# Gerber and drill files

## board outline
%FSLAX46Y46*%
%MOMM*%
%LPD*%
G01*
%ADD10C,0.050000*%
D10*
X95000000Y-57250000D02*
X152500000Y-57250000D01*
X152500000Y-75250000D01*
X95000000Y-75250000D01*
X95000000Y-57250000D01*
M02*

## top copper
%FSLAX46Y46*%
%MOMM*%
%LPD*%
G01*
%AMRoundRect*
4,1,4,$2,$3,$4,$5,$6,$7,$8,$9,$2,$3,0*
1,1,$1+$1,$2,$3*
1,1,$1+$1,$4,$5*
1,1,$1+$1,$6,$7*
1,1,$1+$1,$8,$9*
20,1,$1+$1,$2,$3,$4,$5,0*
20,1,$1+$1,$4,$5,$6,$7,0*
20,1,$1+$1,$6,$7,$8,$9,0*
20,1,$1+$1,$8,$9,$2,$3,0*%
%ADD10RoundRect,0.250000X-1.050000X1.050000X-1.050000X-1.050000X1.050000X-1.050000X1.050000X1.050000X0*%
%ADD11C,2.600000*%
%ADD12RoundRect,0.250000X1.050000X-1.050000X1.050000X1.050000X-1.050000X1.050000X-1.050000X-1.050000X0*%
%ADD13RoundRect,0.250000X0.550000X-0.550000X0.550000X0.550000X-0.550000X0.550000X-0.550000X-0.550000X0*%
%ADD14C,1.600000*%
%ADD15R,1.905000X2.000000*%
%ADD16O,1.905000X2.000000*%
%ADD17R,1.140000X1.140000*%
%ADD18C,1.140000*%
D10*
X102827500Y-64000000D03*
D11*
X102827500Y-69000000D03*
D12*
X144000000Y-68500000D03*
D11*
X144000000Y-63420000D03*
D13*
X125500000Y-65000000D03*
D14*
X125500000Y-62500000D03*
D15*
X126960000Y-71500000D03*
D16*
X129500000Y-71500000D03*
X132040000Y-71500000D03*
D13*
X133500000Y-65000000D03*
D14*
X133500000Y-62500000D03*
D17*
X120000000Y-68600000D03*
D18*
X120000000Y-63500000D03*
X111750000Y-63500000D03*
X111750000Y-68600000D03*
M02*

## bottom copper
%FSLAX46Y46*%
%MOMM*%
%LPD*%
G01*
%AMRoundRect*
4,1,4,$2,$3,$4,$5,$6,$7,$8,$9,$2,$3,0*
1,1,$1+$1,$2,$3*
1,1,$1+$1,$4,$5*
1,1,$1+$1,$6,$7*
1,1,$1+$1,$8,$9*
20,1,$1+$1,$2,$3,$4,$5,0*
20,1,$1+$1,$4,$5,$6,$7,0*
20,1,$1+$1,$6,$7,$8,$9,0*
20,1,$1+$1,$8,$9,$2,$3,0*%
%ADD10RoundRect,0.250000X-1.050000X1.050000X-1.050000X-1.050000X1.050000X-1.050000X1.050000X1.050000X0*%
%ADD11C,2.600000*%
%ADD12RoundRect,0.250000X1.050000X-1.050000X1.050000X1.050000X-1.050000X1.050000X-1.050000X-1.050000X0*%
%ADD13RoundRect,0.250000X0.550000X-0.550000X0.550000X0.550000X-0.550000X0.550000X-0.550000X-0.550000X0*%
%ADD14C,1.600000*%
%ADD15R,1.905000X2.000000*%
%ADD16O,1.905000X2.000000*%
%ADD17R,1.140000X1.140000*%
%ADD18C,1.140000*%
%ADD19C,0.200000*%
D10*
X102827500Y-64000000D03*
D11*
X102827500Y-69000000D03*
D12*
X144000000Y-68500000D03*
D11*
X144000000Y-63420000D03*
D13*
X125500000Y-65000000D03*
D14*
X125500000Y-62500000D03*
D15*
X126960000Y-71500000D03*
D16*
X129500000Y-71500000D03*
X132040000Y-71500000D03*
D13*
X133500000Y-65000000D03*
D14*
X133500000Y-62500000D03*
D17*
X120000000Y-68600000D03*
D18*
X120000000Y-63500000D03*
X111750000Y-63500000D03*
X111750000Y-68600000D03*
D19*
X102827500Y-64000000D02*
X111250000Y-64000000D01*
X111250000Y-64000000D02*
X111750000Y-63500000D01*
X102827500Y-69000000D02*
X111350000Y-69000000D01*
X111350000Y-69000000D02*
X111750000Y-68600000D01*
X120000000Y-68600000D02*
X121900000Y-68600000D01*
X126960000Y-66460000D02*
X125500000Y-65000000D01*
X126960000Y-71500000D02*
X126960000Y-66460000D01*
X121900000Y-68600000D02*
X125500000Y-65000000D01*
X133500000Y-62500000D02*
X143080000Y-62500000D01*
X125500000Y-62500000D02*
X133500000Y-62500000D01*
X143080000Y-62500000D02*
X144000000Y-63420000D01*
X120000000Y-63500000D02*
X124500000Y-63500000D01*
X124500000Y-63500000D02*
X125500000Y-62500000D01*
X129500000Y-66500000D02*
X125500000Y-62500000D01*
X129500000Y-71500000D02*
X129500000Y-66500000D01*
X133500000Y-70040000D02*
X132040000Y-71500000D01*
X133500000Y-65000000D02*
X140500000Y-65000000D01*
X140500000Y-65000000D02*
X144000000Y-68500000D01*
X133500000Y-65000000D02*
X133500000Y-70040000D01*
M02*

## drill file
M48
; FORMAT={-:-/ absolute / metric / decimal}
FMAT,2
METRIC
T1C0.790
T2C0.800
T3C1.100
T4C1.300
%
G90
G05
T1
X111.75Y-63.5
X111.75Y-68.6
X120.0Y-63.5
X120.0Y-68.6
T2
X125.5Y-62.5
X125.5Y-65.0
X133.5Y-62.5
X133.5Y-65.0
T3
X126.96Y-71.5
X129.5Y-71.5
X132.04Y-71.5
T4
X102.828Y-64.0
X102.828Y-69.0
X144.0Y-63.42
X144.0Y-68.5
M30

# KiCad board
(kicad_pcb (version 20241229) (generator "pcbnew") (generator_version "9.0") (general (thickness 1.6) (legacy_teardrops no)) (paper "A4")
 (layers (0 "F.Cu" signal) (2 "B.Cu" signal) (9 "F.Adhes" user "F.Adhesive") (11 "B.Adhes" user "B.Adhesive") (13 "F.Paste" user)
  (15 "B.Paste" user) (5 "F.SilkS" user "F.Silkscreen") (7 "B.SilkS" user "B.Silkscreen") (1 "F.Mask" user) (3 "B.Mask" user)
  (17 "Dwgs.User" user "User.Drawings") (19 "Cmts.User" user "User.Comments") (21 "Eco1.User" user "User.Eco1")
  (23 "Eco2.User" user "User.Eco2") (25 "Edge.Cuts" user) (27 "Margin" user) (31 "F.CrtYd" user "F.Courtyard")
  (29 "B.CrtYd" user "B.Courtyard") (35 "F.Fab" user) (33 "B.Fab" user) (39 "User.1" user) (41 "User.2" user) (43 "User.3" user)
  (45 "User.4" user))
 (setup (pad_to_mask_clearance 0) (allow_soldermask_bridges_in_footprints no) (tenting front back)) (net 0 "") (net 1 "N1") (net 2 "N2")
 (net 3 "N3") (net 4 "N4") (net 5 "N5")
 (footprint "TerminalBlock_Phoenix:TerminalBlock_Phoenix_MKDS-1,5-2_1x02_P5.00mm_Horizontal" (layer "F.Cu") (at 102.8275 64 -90)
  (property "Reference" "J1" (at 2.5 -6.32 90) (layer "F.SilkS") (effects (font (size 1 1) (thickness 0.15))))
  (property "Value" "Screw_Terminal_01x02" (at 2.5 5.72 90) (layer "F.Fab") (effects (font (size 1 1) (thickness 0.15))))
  (pad "1" thru_hole roundrect (at 0 0 270) (size 2.6 2.6) (drill 1.3) (layers "*.Cu" "*.Mask") (remove_unused_layers no)
   (roundrect_rratio 0.096154) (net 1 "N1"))
  (pad "2" thru_hole circle (at 5 0 270) (size 2.6 2.6) (drill 1.3) (layers "*.Cu" "*.Mask") (remove_unused_layers no) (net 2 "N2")))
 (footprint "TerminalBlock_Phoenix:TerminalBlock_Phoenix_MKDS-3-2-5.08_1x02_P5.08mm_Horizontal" (layer "F.Cu") (at 144 68.5 90)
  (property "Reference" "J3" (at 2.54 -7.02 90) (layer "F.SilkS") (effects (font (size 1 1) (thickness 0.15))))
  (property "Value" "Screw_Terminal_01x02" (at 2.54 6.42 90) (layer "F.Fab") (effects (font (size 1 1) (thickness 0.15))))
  (pad "1" thru_hole roundrect (at 0 0 90) (size 2.6 2.6) (drill 1.3) (layers "*.Cu" "*.Mask") (remove_unused_layers no)
   (roundrect_rratio 0.096154) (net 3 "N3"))
  (pad "2" thru_hole circle (at 5.08 0 90) (size 2.6 2.6) (drill 1.3) (layers "*.Cu" "*.Mask") (remove_unused_layers no) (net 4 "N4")))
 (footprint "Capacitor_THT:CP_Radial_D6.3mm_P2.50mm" (layer "F.Cu") (at 125.5 65 90)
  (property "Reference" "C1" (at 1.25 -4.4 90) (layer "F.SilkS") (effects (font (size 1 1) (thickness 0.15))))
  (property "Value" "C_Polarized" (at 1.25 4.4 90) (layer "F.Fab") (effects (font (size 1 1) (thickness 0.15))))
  (pad "1" thru_hole roundrect (at 0 0 90) (size 1.6 1.6) (drill 0.8) (layers "*.Cu" "*.Mask") (remove_unused_layers no)
   (roundrect_rratio 0.15625) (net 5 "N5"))
  (pad "2" thru_hole circle (at 2.5 0 90) (size 1.6 1.6) (drill 0.8) (layers "*.Cu" "*.Mask") (remove_unused_layers no) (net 4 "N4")))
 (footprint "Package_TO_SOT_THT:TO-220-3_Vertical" (layer "F.Cu") (at 126.96 71.5)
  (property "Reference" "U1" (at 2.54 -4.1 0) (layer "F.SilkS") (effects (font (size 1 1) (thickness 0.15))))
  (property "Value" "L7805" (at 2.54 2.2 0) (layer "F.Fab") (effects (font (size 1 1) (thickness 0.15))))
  (pad "1" thru_hole rect (at 0 0) (size 1.905 2) (drill 1.1) (layers "*.Cu" "*.Mask") (remove_unused_layers no) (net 5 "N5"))
  (pad "2" thru_hole oval (at 2.54 0) (size 1.905 2) (drill 1.1) (layers "*.Cu" "*.Mask") (remove_unused_layers no) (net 4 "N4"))
  (pad "3" thru_hole oval (at 5.08 0) (size 1.905 2) (drill 1.1) (layers "*.Cu" "*.Mask") (remove_unused_layers no) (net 3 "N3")))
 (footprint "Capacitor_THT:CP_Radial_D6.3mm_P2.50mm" (layer "F.Cu") (at 133.5 65 90)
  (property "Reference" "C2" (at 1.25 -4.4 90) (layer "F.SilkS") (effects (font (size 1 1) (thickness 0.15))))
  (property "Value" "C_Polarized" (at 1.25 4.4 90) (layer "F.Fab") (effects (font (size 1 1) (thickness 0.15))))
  (pad "1" thru_hole roundrect (at 0 0 90) (size 1.6 1.6) (drill 0.8) (layers "*.Cu" "*.Mask") (remove_unused_layers no)
   (roundrect_rratio 0.15625) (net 3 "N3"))
  (pad "2" thru_hole circle (at 2.5 0 90) (size 1.6 1.6) (drill 0.8) (layers "*.Cu" "*.Mask") (remove_unused_layers no) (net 4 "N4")))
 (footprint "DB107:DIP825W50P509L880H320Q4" (layer "F.Cu") (at 115.875 66.05 180)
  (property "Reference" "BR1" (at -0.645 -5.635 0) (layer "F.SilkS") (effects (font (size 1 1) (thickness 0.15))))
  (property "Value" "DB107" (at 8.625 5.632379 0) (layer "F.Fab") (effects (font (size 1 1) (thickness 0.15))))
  (pad "1" thru_hole rect (at -4.125 -2.55 180) (size 1.14 1.14) (drill 0.79) (layers "*.Cu" "*.Mask") (remove_unused_layers no)
   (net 5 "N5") (solder_mask_margin 0.102))
  (pad "2" thru_hole circle (at -4.125 2.55 180) (size 1.14 1.14) (drill 0.79) (layers "*.Cu" "*.Mask") (remove_unused_layers no)
   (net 4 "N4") (solder_mask_margin 0.102))
  (pad "3" thru_hole circle (at 4.125 2.55 180) (size 1.14 1.14) (drill 0.79) (layers "*.Cu" "*.Mask") (remove_unused_layers no)
   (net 1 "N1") (solder_mask_margin 0.102))
  (pad "4" thru_hole circle (at 4.125 -2.55 180) (size 1.14 1.14) (drill 0.79) (layers "*.Cu" "*.Mask") (remove_unused_layers no)
   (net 2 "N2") (solder_mask_margin 0.102)))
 (gr_rect (start 95 57.25) (end 152.5 75.25) (stroke (width 0.05) (type default)) (fill no) (layer "Edge.Cuts"))
 (segment (start 102.8275 64) (end 111.25 64) (width 0.2) (layer "B.Cu") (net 1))
 (segment (start 111.25 64) (end 111.75 63.5) (width 0.2) (layer "B.Cu") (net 1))
 (segment (start 102.8275 69) (end 111.35 69) (width 0.2) (layer "B.Cu") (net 2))
 (segment (start 111.35 69) (end 111.75 68.6) (width 0.2) (layer "B.Cu") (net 2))
 (segment (start 120 68.6) (end 121.9 68.6) (width 0.2) (layer "B.Cu") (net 5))
 (segment (start 126.96 66.46) (end 125.5 65) (width 0.2) (layer "B.Cu") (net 5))
 (segment (start 126.96 71.5) (end 126.96 66.46) (width 0.2) (layer "B.Cu") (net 5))
 (segment (start 121.9 68.6) (end 125.5 65) (width 0.2) (layer "B.Cu") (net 5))
 (segment (start 133.5 62.5) (end 143.08 62.5) (width 0.2) (layer "B.Cu") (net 4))
 (segment (start 125.5 62.5) (end 133.5 62.5) (width 0.2) (layer "B.Cu") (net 4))
 (segment (start 143.08 62.5) (end 144 63.42) (width 0.2) (layer "B.Cu") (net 4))
 (segment (start 120 63.5) (end 124.5 63.5) (width 0.2) (layer "B.Cu") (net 4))
 (segment (start 124.5 63.5) (end 125.5 62.5) (width 0.2) (layer "B.Cu") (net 4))
 (segment (start 129.5 66.5) (end 125.5 62.5) (width 0.2) (layer "B.Cu") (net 4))
 (segment (start 129.5 71.5) (end 129.5 66.5) (width 0.2) (layer "B.Cu") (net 4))
 (segment (start 133.5 70.04) (end 132.04 71.5) (width 0.2) (layer "B.Cu") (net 3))
 (segment (start 133.5 65) (end 140.5 65) (width 0.2) (layer "B.Cu") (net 3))
 (segment (start 140.5 65) (end 144 68.5) (width 0.2) (layer "B.Cu") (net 3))
 (segment (start 133.5 65) (end 133.5 70.04) (width 0.2) (layer "B.Cu") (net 3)))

